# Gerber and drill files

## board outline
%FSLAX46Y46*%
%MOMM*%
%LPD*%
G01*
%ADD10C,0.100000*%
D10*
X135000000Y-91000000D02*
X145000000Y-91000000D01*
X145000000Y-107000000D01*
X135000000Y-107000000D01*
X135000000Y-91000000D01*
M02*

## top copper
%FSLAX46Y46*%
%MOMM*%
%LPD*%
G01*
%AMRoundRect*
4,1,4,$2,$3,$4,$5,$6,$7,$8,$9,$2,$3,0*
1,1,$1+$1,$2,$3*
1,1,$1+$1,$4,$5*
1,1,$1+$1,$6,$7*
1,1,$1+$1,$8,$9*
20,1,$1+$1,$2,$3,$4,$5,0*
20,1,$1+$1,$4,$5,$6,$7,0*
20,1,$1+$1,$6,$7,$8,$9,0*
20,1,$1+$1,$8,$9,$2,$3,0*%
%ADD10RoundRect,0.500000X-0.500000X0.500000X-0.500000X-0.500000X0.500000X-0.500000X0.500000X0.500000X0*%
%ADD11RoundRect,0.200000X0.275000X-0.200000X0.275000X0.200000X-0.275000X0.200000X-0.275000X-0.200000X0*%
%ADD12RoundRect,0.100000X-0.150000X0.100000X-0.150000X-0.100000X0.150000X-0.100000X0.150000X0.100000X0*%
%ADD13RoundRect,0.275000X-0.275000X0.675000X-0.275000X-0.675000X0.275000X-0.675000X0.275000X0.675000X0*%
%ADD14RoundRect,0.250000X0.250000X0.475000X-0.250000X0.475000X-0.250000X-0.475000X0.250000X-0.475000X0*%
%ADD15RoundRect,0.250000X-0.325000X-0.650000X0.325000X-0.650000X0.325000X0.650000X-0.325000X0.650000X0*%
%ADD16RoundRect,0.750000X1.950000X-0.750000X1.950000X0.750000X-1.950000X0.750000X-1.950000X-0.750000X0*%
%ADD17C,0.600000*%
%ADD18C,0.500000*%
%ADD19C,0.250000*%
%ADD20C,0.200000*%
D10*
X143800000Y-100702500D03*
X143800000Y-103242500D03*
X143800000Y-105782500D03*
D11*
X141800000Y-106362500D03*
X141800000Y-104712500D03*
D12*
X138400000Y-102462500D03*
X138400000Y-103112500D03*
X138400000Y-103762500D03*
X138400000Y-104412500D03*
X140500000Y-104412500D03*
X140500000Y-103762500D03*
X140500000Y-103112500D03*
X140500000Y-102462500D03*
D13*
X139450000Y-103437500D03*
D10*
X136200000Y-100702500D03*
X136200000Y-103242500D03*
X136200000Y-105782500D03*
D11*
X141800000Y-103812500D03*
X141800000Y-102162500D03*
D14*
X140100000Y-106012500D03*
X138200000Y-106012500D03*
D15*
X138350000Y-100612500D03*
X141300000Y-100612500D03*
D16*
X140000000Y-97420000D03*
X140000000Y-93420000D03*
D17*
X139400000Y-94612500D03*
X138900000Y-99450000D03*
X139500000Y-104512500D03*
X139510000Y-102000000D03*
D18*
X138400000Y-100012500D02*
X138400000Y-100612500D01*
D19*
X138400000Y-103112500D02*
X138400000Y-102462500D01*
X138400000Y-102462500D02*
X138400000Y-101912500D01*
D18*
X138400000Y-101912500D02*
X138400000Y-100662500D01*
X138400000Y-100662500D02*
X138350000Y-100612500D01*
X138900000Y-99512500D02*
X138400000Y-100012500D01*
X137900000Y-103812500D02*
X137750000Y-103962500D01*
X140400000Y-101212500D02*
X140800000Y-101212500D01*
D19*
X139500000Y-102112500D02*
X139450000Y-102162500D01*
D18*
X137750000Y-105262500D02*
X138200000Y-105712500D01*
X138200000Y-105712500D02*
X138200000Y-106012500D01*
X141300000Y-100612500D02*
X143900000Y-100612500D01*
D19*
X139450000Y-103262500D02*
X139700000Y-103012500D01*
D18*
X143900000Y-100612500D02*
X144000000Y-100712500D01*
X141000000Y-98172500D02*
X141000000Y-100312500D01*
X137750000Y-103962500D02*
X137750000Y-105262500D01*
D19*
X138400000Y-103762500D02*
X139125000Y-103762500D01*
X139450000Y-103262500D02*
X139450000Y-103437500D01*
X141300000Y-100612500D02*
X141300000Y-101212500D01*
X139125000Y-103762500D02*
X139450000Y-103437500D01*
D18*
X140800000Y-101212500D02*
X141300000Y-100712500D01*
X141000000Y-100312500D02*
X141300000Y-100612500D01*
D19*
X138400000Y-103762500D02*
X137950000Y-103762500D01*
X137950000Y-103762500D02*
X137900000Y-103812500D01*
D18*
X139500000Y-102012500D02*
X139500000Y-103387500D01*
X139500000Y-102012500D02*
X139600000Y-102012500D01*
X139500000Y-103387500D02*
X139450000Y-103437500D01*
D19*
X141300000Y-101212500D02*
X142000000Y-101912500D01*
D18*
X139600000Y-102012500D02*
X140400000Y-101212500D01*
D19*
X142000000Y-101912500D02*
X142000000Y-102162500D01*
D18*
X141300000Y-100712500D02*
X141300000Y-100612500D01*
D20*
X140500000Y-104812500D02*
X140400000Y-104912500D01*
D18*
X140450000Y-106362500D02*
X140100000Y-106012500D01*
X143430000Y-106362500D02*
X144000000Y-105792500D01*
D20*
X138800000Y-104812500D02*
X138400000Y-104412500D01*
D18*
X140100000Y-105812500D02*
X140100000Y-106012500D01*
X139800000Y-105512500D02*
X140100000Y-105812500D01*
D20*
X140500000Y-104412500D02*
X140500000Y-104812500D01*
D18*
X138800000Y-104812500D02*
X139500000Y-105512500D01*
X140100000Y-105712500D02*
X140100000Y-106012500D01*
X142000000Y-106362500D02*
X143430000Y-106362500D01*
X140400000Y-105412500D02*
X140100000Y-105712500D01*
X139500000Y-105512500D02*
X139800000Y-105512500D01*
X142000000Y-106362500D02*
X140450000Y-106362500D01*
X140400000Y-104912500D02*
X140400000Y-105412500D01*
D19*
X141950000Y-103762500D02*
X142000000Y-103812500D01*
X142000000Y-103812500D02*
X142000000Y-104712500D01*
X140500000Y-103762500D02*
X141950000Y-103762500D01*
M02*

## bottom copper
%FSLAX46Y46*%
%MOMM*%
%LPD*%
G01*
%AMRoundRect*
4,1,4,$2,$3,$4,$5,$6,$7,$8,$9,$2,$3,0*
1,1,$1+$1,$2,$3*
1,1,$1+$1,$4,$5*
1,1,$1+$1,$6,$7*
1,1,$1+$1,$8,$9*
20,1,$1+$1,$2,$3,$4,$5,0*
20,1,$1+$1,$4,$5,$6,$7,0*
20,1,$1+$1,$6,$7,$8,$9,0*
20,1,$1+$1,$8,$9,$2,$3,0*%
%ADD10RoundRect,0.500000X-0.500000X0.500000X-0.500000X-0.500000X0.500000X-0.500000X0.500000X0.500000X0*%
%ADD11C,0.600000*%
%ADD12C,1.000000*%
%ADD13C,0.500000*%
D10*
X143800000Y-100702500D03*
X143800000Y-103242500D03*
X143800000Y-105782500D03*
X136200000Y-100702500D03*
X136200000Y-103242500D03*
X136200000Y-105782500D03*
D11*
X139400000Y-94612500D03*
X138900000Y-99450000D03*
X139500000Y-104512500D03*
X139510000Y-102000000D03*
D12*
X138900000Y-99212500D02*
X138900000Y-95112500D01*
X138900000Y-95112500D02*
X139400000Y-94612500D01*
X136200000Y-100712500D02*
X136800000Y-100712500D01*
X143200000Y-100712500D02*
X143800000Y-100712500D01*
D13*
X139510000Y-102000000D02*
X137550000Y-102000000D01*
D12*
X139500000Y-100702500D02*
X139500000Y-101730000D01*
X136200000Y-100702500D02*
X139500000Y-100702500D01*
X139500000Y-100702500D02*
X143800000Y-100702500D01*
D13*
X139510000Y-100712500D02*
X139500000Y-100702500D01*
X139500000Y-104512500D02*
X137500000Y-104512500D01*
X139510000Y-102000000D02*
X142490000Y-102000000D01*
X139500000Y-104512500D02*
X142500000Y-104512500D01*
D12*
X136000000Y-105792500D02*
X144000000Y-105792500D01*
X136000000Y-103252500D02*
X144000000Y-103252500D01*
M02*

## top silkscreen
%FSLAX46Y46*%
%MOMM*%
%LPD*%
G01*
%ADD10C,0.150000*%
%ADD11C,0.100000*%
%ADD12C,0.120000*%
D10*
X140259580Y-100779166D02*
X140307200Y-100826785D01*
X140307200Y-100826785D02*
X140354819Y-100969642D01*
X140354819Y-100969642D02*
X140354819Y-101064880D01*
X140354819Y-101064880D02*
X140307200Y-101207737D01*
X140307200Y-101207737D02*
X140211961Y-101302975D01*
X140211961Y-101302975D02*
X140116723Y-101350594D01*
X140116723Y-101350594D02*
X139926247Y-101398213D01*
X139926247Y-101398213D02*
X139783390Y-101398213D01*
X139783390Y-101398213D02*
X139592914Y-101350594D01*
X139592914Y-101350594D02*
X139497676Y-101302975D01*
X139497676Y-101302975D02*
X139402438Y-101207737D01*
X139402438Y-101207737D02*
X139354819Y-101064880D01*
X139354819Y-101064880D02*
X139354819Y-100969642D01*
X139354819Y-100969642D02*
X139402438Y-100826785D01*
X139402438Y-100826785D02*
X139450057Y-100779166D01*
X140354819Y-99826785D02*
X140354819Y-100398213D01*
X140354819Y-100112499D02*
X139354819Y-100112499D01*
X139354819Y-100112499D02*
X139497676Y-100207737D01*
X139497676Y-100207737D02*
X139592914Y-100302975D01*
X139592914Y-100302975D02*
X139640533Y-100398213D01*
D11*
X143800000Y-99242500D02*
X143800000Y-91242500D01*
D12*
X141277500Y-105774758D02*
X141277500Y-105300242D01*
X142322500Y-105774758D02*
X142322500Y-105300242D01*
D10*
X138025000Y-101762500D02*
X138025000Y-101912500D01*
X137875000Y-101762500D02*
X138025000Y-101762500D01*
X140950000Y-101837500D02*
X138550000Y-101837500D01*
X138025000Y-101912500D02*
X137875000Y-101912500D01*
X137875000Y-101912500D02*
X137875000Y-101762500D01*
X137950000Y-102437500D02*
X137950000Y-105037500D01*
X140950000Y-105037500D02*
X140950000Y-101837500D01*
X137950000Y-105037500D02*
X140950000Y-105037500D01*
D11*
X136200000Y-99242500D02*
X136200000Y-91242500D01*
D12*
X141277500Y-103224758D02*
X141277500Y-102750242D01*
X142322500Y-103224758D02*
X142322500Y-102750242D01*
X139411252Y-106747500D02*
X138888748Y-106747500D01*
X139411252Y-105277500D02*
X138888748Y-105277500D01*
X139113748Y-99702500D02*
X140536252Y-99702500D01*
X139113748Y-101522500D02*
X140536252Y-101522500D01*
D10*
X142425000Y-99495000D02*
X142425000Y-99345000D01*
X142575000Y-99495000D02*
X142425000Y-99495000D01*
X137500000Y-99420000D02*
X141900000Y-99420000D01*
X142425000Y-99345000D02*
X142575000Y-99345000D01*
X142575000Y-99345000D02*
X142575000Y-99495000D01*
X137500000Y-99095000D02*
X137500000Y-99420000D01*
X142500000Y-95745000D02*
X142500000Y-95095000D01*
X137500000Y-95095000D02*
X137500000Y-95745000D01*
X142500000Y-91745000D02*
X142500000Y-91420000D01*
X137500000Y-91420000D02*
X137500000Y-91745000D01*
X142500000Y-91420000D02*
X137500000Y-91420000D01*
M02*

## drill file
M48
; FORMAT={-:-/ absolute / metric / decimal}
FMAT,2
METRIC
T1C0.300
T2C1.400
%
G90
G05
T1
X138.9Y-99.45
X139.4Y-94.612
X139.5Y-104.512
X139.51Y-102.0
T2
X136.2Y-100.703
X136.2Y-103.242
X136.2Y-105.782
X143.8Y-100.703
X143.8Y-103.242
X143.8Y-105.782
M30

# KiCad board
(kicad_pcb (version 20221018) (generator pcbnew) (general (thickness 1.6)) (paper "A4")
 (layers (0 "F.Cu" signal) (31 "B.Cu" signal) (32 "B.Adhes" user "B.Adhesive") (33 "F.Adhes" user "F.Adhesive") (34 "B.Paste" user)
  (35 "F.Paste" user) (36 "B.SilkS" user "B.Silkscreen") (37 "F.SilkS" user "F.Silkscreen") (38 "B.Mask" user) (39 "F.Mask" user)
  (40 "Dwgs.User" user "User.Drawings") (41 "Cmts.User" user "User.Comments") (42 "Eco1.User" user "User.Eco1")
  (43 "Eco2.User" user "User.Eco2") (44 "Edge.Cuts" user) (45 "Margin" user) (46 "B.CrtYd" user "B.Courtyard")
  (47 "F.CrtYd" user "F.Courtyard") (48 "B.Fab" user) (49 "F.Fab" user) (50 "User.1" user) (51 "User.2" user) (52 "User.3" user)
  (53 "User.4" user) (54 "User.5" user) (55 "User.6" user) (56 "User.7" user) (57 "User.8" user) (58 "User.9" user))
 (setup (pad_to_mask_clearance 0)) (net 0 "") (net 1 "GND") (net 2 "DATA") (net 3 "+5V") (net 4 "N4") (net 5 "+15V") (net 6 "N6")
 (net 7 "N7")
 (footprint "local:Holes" (layer "F.Cu") (at 143.8 103.2425 -90)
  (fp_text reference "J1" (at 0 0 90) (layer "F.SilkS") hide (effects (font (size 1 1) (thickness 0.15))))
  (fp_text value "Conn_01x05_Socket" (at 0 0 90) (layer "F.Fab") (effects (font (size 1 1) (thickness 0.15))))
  (fp_line (start -4 0) (end -12 0) (stroke (width 0.1) (type solid)) (layer "F.SilkS"))
  (pad "1" thru_hole roundrect (at -2.54 0 270) (size 2 2) (drill 1.4) (layers "*.Cu" "*.Mask") (roundrect_rratio 0.25) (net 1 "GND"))
  (pad "2" thru_hole roundrect (at 0 0 270) (size 2 2) (drill 1.4) (layers "*.Cu" "*.Mask") (roundrect_rratio 0.25) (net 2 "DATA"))
  (pad "3" thru_hole roundrect (at 2.54 0 270) (size 2 2) (drill 1.4) (layers "*.Cu" "*.Mask") (roundrect_rratio 0.25) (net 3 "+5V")))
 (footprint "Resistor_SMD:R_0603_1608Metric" (layer "F.Cu") (at 141.8 105.5375 90)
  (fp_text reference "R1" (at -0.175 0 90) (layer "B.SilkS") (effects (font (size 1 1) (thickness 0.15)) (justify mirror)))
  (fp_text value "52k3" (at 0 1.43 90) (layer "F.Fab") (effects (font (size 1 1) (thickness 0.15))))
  (fp_line (start -0.237258 -0.5225) (end 0.237258 -0.5225) (stroke (width 0.12) (type solid)) (layer "F.SilkS"))
  (fp_line (start -0.237258 0.5225) (end 0.237258 0.5225) (stroke (width 0.12) (type solid)) (layer "F.SilkS"))
  (pad "1" smd roundrect (at -0.825 0 90) (size 0.8 0.95) (layers "F.Cu" "F.Paste" "F.Mask") (roundrect_rratio 0.25) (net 3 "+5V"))
  (pad "2" smd roundrect (at 0.825 0 90) (size 0.8 0.95) (layers "F.Cu" "F.Paste" "F.Mask") (roundrect_rratio 0.25) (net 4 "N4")))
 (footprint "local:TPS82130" (layer "F.Cu") (at 139.45 103.4375 -90)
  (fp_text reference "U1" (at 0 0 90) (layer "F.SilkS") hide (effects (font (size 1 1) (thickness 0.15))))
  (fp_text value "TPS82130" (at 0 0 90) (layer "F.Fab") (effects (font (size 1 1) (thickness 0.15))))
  (fp_line (start -1.675 1.425) (end -1.525 1.425) (stroke (width 0.15) (type solid)) (layer "F.SilkS"))
  (fp_line (start -1.675 1.575) (end -1.675 1.425) (stroke (width 0.15) (type solid)) (layer "F.SilkS"))
  (fp_line (start -1.6 -1.5) (end -1.6 0.9) (stroke (width 0.15) (type solid)) (layer "F.SilkS"))
  (fp_line (start -1.525 1.425) (end -1.525 1.575) (stroke (width 0.15) (type solid)) (layer "F.SilkS"))
  (fp_line (start -1.525 1.575) (end -1.675 1.575) (stroke (width 0.15) (type solid)) (layer "F.SilkS"))
  (fp_line (start -1 1.5) (end 1.6 1.5) (stroke (width 0.15) (type solid)) (layer "F.SilkS"))
  (fp_line (start 1.6 -1.5) (end -1.6 -1.5) (stroke (width 0.15) (type solid)) (layer "F.SilkS"))
  (fp_line (start 1.6 1.5) (end 1.6 -1.5) (stroke (width 0.15) (type solid)) (layer "F.SilkS"))
  (pad "1" smd roundrect (at -0.975 1.05 270) (size 0.4 0.5) (layers "F.Cu" "F.Paste" "F.Mask") (roundrect_rratio 0.25) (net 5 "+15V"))
  (pad "2" smd roundrect (at -0.325 1.05 270) (size 0.4 0.5) (layers "F.Cu" "F.Paste" "F.Mask") (roundrect_rratio 0.25) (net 5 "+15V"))
  (pad "3" smd roundrect (at 0.325 1.05 270) (size 0.4 0.5) (layers "F.Cu" "F.Paste" "F.Mask") (roundrect_rratio 0.25) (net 1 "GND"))
  (pad "4" smd roundrect (at 0.975 1.05 270) (size 0.4 0.5) (layers "F.Cu" "F.Paste" "F.Mask") (roundrect_rratio 0.25) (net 3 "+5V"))
  (pad "5" smd roundrect (at 0.975 -1.05 270) (size 0.4 0.5) (layers "F.Cu" "F.Paste" "F.Mask") (roundrect_rratio 0.25) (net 3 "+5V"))
  (pad "6" smd roundrect (at 0.325 -1.05 270) (size 0.4 0.5) (layers "F.Cu" "F.Paste" "F.Mask") (roundrect_rratio 0.25) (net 4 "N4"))
  (pad "7" smd roundrect (at -0.325 -1.05 270) (size 0.4 0.5) (layers "F.Cu" "F.Paste" "F.Mask") (roundrect_rratio 0.25) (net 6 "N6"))
  (pad "8" smd roundrect (at -0.975 -1.05 270) (size 0.4 0.5) (layers "F.Cu" "F.Paste" "F.Mask") (roundrect_rratio 0.25) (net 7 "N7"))
  (pad "9" smd roundrect (at 0 0 270) (size 1.9 1.1) (layers "F.Cu" "F.Paste" "F.Mask") (roundrect_rratio 0.25) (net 1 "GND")))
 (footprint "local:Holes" (layer "F.Cu") (at 136.2 103.2425 -90)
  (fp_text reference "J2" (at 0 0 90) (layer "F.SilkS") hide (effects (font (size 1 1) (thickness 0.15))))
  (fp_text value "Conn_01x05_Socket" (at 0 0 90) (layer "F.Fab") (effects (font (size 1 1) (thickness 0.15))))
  (fp_line (start -4 0) (end -12 0) (stroke (width 0.1) (type solid)) (layer "F.SilkS"))
  (pad "1" thru_hole roundrect (at -2.54 0 270) (size 2 2) (drill 1.4) (layers "*.Cu" "*.Mask") (roundrect_rratio 0.25) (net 1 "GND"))
  (pad "2" thru_hole roundrect (at 0 0 270) (size 2 2) (drill 1.4) (layers "*.Cu" "*.Mask") (roundrect_rratio 0.25) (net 2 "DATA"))
  (pad "3" thru_hole roundrect (at 2.54 0 270) (size 2 2) (drill 1.4) (layers "*.Cu" "*.Mask") (roundrect_rratio 0.25) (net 3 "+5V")))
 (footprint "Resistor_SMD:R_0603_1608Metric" (layer "F.Cu") (at 141.8 102.9875 90)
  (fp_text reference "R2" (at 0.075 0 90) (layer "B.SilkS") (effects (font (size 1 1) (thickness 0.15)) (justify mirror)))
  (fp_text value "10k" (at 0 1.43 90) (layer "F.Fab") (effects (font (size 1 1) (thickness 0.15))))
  (fp_line (start -0.237258 -0.5225) (end 0.237258 -0.5225) (stroke (width 0.12) (type solid)) (layer "F.SilkS"))
  (fp_line (start -0.237258 0.5225) (end 0.237258 0.5225) (stroke (width 0.12) (type solid)) (layer "F.SilkS"))
  (pad "1" smd roundrect (at -0.825 0 90) (size 0.8 0.95) (layers "F.Cu" "F.Paste" "F.Mask") (roundrect_rratio 0.25) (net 4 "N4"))
  (pad "2" smd roundrect (at 0.825 0 90) (size 0.8 0.95) (layers "F.Cu" "F.Paste" "F.Mask") (roundrect_rratio 0.25) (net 1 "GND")))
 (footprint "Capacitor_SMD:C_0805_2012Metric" (layer "F.Cu") (at 139.15 106.0125 180)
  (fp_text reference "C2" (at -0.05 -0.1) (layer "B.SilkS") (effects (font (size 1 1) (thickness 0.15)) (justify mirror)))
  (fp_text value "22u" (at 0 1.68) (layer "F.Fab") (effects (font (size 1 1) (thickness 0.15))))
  (fp_line (start -0.261252 -0.735) (end 0.261252 -0.735) (stroke (width 0.12) (type solid)) (layer "F.SilkS"))
  (fp_line (start -0.261252 0.735) (end 0.261252 0.735) (stroke (width 0.12) (type solid)) (layer "F.SilkS"))
  (pad "1" smd roundrect (at -0.95 0 180) (size 1 1.45) (layers "F.Cu" "F.Paste" "F.Mask") (roundrect_rratio 0.25) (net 3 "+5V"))
  (pad "2" smd roundrect (at 0.95 0 180) (size 1 1.45) (layers "F.Cu" "F.Paste" "F.Mask") (roundrect_rratio 0.25) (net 1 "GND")))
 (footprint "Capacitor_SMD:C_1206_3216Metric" (layer "F.Cu") (at 139.825 100.6125)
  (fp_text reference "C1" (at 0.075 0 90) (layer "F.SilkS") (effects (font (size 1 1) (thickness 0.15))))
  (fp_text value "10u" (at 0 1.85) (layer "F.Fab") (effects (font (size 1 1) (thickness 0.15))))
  (fp_line (start -0.711252 -0.91) (end 0.711252 -0.91) (stroke (width 0.12) (type solid)) (layer "F.SilkS"))
  (fp_line (start -0.711252 0.91) (end 0.711252 0.91) (stroke (width 0.12) (type solid)) (layer "F.SilkS"))
  (pad "1" smd roundrect (at -1.475 0) (size 1.15 1.8) (layers "F.Cu" "F.Paste" "F.Mask") (roundrect_rratio 0.217391) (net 5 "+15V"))
  (pad "2" smd roundrect (at 1.475 0) (size 1.15 1.8) (layers "F.Cu" "F.Paste" "F.Mask") (roundrect_rratio 0.217391) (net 1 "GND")))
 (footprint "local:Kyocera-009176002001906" (layer "F.Cu") (at 140 95.42 90)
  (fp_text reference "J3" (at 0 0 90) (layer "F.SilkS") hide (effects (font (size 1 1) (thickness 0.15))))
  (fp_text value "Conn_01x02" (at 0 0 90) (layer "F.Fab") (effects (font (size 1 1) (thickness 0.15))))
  (fp_line (start -4.075 2.425) (end -3.925 2.425) (stroke (width 0.15) (type solid)) (layer "F.SilkS"))
  (fp_line (start -4.075 2.575) (end -4.075 2.425) (stroke (width 0.15) (type solid)) (layer "F.SilkS"))
  (fp_line (start -4 -2.5) (end -4 1.9) (stroke (width 0.15) (type solid)) (layer "F.SilkS"))
  (fp_line (start -3.925 2.425) (end -3.925 2.575) (stroke (width 0.15) (type solid)) (layer "F.SilkS"))
  (fp_line (start -3.925 2.575) (end -4.075 2.575) (stroke (width 0.15) (type solid)) (layer "F.SilkS"))
  (fp_line (start -3.675 -2.5) (end -4 -2.5) (stroke (width 0.15) (type solid)) (layer "F.SilkS"))
  (fp_line (start -0.325 2.5) (end 0.325 2.5) (stroke (width 0.15) (type solid)) (layer "F.SilkS"))
  (fp_line (start 0.325 -2.5) (end -0.325 -2.5) (stroke (width 0.15) (type solid)) (layer "F.SilkS"))
  (fp_line (start 3.675 2.5) (end 4 2.5) (stroke (width 0.15) (type solid)) (layer "F.SilkS"))
  (fp_line (start 4 -2.5) (end 3.675 -2.5) (stroke (width 0.15) (type solid)) (layer "F.SilkS"))
  (fp_line (start 4 2.5) (end 4 -2.5) (stroke (width 0.15) (type solid)) (layer "F.SilkS"))
  (pad "1" smd roundrect (at -2 0 90) (size 3 5.4) (layers "F.Cu" "F.Paste" "F.Mask") (roundrect_rratio 0.25) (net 1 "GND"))
  (pad "2" smd roundrect (at 2 0 90) (size 3 5.4) (layers "F.Cu" "F.Paste" "F.Mask") (roundrect_rratio 0.25) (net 5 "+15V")))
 (gr_rect (start 135 91) (end 145 107) (stroke (width 0.1) (type default)) (fill none) (layer "Edge.Cuts"))
 (segment (start 138.4 100.0125) (end 138.4 100.6125) (width 0.5) (layer "F.Cu") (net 5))
 (segment (start 138.4 103.1125) (end 138.4 102.4625) (width 0.25) (layer "F.Cu") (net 5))
 (segment (start 138.4 102.4625) (end 138.4 101.9125) (width 0.25) (layer "F.Cu") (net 5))
 (segment (start 138.4 101.9125) (end 138.4 100.6625) (width 0.5) (layer "F.Cu") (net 5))
 (segment (start 138.4 100.6625) (end 138.35 100.6125) (width 0.5) (layer "F.Cu") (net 5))
 (segment (start 138.9 99.5125) (end 138.4 100.0125) (width 0.5) (layer "F.Cu") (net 5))
 (via (at 139.4 94.6125) (size 0.6) (drill 0.3) (layers "F.Cu" "B.Cu") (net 5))
 (via (at 138.9 99.45) (size 0.6) (drill 0.3) (layers "F.Cu" "B.Cu") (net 5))
 (segment (start 138.9 99.2125) (end 138.9 95.1125) (width 1) (layer "B.Cu") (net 5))
 (segment (start 138.9 95.1125) (end 139.4 94.6125) (width 1) (layer "B.Cu") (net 5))
 (segment (start 137.9 103.8125) (end 137.75 103.9625) (width 0.5) (layer "F.Cu") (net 1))
 (segment (start 140.4 101.2125) (end 140.8 101.2125) (width 0.5) (layer "F.Cu") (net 1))
 (segment (start 139.5 102.1125) (end 139.45 102.1625) (width 0.25) (layer "F.Cu") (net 1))
 (segment (start 137.75 105.2625) (end 138.2 105.7125) (width 0.5) (layer "F.Cu") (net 1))
 (segment (start 138.2 105.7125) (end 138.2 106.0125) (width 0.5) (layer "F.Cu") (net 1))
 (segment (start 141.3 100.6125) (end 143.9 100.6125) (width 0.5) (layer "F.Cu") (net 1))
 (segment (start 139.45 103.2625) (end 139.7 103.0125) (width 0.25) (layer "F.Cu") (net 1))
 (segment (start 143.9 100.6125) (end 144 100.7125) (width 0.5) (layer "F.Cu") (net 1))
 (segment (start 141 98.1725) (end 141 100.3125) (width 0.5) (layer "F.Cu") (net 1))
 (segment (start 137.75 103.9625) (end 137.75 105.2625) (width 0.5) (layer "F.Cu") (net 1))
 (segment (start 138.4 103.7625) (end 139.125 103.7625) (width 0.25) (layer "F.Cu") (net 1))
 (segment (start 139.45 103.2625) (end 139.45 103.4375) (width 0.25) (layer "F.Cu") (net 1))
 (segment (start 141.3 100.6125) (end 141.3 101.2125) (width 0.25) (layer "F.Cu") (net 1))
 (segment (start 139.125 103.7625) (end 139.45 103.4375) (width 0.25) (layer "F.Cu") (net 1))
 (segment (start 140.8 101.2125) (end 141.3 100.7125) (width 0.5) (layer "F.Cu") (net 1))
 (segment (start 141 100.3125) (end 141.3 100.6125) (width 0.5) (layer "F.Cu") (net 1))
 (segment (start 138.4 103.7625) (end 137.95 103.7625) (width 0.25) (layer "F.Cu") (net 1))
 (segment (start 137.95 103.7625) (end 137.9 103.8125) (width 0.25) (layer "F.Cu") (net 1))
 (segment (start 139.5 102.0125) (end 139.5 103.3875) (width 0.5) (layer "F.Cu") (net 1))
 (segment (start 139.5 102.0125) (end 139.6 102.0125) (width 0.5) (layer "F.Cu") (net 1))
 (segment (start 139.5 103.3875) (end 139.45 103.4375) (width 0.5) (layer "F.Cu") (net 1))
 (segment (start 141.3 101.2125) (end 142 101.9125) (width 0.25) (layer "F.Cu") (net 1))
 (segment (start 139.6 102.0125) (end 140.4 101.2125) (width 0.5) (layer "F.Cu") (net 1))
 (segment (start 142 101.9125) (end 142 102.1625) (width 0.25) (layer "F.Cu") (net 1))
 (segment (start 141.3 100.7125) (end 141.3 100.6125) (width 0.5) (layer "F.Cu") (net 1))
 (via (at 139.5 104.5125) (size 0.6) (drill 0.3) (layers "F.Cu" "B.Cu") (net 1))
 (via (at 139.51 102) (size 0.6) (drill 0.3) (layers "F.Cu" "B.Cu") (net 1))
 (segment (start 136.2 100.7125) (end 136.8 100.7125) (width 1) (layer "B.Cu") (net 1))
 (segment (start 143.2 100.7125) (end 143.8 100.7125) (width 1) (layer "B.Cu") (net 1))
 (segment (start 139.51 102) (end 137.55 102) (width 0.5) (layer "B.Cu") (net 1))
 (segment (start 139.5 100.7025) (end 139.5 101.73) (width 1) (layer "B.Cu") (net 1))
 (segment (start 136.2 100.7025) (end 139.5 100.7025) (width 1) (layer "B.Cu") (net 1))
 (segment (start 139.5 100.7025) (end 143.8 100.7025) (width 1) (layer "B.Cu") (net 1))
 (segment (start 139.51 100.7125) (end 139.5 100.7025) (width 0.5) (layer "B.Cu") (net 1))
 (segment (start 139.5 104.5125) (end 137.5 104.5125) (width 0.5) (layer "B.Cu") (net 1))
 (segment (start 139.51 102) (end 142.49 102) (width 0.5) (layer "B.Cu") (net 1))
 (segment (start 139.5 104.5125) (end 142.5 104.5125) (width 0.5) (layer "B.Cu") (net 1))
 (segment (start 140.5 104.8125) (end 140.4 104.9125) (width 0.2) (layer "F.Cu") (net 3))
 (segment (start 140.45 106.3625) (end 140.1 106.0125) (width 0.5) (layer "F.Cu") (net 3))
 (segment (start 143.43 106.3625) (end 144 105.7925) (width 0.5) (layer "F.Cu") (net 3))
 (segment (start 138.8 104.8125) (end 138.4 104.4125) (width 0.2) (layer "F.Cu") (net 3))
 (segment (start 140.1 105.8125) (end 140.1 106.0125) (width 0.5) (layer "F.Cu") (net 3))
 (segment (start 139.8 105.5125) (end 140.1 105.8125) (width 0.5) (layer "F.Cu") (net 3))
 (segment (start 140.5 104.4125) (end 140.5 104.8125) (width 0.2) (layer "F.Cu") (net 3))
 (segment (start 138.8 104.8125) (end 139.5 105.5125) (width 0.5) (layer "F.Cu") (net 3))
 (segment (start 140.1 105.7125) (end 140.1 106.0125) (width 0.5) (layer "F.Cu") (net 3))
 (segment (start 142 106.3625) (end 143.43 106.3625) (width 0.5) (layer "F.Cu") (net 3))
 (segment (start 140.4 105.4125) (end 140.1 105.7125) (width 0.5) (layer "F.Cu") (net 3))
 (segment (start 139.5 105.5125) (end 139.8 105.5125) (width 0.5) (layer "F.Cu") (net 3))
 (segment (start 142 106.3625) (end 140.45 106.3625) (width 0.5) (layer "F.Cu") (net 3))
 (segment (start 140.4 104.9125) (end 140.4 105.4125) (width 0.5) (layer "F.Cu") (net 3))
 (segment (start 136 105.7925) (end 144 105.7925) (width 1) (layer "B.Cu") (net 3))
 (segment (start 141.95 103.7625) (end 142 103.8125) (width 0.25) (layer "F.Cu") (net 4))
 (segment (start 142 103.8125) (end 142 104.7125) (width 0.25) (layer "F.Cu") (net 4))
 (segment (start 140.5 103.7625) (end 141.95 103.7625) (width 0.25) (layer "F.Cu") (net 4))
 (segment (start 136 103.2525) (end 144 103.2525) (width 1) (layer "B.Cu") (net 2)))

